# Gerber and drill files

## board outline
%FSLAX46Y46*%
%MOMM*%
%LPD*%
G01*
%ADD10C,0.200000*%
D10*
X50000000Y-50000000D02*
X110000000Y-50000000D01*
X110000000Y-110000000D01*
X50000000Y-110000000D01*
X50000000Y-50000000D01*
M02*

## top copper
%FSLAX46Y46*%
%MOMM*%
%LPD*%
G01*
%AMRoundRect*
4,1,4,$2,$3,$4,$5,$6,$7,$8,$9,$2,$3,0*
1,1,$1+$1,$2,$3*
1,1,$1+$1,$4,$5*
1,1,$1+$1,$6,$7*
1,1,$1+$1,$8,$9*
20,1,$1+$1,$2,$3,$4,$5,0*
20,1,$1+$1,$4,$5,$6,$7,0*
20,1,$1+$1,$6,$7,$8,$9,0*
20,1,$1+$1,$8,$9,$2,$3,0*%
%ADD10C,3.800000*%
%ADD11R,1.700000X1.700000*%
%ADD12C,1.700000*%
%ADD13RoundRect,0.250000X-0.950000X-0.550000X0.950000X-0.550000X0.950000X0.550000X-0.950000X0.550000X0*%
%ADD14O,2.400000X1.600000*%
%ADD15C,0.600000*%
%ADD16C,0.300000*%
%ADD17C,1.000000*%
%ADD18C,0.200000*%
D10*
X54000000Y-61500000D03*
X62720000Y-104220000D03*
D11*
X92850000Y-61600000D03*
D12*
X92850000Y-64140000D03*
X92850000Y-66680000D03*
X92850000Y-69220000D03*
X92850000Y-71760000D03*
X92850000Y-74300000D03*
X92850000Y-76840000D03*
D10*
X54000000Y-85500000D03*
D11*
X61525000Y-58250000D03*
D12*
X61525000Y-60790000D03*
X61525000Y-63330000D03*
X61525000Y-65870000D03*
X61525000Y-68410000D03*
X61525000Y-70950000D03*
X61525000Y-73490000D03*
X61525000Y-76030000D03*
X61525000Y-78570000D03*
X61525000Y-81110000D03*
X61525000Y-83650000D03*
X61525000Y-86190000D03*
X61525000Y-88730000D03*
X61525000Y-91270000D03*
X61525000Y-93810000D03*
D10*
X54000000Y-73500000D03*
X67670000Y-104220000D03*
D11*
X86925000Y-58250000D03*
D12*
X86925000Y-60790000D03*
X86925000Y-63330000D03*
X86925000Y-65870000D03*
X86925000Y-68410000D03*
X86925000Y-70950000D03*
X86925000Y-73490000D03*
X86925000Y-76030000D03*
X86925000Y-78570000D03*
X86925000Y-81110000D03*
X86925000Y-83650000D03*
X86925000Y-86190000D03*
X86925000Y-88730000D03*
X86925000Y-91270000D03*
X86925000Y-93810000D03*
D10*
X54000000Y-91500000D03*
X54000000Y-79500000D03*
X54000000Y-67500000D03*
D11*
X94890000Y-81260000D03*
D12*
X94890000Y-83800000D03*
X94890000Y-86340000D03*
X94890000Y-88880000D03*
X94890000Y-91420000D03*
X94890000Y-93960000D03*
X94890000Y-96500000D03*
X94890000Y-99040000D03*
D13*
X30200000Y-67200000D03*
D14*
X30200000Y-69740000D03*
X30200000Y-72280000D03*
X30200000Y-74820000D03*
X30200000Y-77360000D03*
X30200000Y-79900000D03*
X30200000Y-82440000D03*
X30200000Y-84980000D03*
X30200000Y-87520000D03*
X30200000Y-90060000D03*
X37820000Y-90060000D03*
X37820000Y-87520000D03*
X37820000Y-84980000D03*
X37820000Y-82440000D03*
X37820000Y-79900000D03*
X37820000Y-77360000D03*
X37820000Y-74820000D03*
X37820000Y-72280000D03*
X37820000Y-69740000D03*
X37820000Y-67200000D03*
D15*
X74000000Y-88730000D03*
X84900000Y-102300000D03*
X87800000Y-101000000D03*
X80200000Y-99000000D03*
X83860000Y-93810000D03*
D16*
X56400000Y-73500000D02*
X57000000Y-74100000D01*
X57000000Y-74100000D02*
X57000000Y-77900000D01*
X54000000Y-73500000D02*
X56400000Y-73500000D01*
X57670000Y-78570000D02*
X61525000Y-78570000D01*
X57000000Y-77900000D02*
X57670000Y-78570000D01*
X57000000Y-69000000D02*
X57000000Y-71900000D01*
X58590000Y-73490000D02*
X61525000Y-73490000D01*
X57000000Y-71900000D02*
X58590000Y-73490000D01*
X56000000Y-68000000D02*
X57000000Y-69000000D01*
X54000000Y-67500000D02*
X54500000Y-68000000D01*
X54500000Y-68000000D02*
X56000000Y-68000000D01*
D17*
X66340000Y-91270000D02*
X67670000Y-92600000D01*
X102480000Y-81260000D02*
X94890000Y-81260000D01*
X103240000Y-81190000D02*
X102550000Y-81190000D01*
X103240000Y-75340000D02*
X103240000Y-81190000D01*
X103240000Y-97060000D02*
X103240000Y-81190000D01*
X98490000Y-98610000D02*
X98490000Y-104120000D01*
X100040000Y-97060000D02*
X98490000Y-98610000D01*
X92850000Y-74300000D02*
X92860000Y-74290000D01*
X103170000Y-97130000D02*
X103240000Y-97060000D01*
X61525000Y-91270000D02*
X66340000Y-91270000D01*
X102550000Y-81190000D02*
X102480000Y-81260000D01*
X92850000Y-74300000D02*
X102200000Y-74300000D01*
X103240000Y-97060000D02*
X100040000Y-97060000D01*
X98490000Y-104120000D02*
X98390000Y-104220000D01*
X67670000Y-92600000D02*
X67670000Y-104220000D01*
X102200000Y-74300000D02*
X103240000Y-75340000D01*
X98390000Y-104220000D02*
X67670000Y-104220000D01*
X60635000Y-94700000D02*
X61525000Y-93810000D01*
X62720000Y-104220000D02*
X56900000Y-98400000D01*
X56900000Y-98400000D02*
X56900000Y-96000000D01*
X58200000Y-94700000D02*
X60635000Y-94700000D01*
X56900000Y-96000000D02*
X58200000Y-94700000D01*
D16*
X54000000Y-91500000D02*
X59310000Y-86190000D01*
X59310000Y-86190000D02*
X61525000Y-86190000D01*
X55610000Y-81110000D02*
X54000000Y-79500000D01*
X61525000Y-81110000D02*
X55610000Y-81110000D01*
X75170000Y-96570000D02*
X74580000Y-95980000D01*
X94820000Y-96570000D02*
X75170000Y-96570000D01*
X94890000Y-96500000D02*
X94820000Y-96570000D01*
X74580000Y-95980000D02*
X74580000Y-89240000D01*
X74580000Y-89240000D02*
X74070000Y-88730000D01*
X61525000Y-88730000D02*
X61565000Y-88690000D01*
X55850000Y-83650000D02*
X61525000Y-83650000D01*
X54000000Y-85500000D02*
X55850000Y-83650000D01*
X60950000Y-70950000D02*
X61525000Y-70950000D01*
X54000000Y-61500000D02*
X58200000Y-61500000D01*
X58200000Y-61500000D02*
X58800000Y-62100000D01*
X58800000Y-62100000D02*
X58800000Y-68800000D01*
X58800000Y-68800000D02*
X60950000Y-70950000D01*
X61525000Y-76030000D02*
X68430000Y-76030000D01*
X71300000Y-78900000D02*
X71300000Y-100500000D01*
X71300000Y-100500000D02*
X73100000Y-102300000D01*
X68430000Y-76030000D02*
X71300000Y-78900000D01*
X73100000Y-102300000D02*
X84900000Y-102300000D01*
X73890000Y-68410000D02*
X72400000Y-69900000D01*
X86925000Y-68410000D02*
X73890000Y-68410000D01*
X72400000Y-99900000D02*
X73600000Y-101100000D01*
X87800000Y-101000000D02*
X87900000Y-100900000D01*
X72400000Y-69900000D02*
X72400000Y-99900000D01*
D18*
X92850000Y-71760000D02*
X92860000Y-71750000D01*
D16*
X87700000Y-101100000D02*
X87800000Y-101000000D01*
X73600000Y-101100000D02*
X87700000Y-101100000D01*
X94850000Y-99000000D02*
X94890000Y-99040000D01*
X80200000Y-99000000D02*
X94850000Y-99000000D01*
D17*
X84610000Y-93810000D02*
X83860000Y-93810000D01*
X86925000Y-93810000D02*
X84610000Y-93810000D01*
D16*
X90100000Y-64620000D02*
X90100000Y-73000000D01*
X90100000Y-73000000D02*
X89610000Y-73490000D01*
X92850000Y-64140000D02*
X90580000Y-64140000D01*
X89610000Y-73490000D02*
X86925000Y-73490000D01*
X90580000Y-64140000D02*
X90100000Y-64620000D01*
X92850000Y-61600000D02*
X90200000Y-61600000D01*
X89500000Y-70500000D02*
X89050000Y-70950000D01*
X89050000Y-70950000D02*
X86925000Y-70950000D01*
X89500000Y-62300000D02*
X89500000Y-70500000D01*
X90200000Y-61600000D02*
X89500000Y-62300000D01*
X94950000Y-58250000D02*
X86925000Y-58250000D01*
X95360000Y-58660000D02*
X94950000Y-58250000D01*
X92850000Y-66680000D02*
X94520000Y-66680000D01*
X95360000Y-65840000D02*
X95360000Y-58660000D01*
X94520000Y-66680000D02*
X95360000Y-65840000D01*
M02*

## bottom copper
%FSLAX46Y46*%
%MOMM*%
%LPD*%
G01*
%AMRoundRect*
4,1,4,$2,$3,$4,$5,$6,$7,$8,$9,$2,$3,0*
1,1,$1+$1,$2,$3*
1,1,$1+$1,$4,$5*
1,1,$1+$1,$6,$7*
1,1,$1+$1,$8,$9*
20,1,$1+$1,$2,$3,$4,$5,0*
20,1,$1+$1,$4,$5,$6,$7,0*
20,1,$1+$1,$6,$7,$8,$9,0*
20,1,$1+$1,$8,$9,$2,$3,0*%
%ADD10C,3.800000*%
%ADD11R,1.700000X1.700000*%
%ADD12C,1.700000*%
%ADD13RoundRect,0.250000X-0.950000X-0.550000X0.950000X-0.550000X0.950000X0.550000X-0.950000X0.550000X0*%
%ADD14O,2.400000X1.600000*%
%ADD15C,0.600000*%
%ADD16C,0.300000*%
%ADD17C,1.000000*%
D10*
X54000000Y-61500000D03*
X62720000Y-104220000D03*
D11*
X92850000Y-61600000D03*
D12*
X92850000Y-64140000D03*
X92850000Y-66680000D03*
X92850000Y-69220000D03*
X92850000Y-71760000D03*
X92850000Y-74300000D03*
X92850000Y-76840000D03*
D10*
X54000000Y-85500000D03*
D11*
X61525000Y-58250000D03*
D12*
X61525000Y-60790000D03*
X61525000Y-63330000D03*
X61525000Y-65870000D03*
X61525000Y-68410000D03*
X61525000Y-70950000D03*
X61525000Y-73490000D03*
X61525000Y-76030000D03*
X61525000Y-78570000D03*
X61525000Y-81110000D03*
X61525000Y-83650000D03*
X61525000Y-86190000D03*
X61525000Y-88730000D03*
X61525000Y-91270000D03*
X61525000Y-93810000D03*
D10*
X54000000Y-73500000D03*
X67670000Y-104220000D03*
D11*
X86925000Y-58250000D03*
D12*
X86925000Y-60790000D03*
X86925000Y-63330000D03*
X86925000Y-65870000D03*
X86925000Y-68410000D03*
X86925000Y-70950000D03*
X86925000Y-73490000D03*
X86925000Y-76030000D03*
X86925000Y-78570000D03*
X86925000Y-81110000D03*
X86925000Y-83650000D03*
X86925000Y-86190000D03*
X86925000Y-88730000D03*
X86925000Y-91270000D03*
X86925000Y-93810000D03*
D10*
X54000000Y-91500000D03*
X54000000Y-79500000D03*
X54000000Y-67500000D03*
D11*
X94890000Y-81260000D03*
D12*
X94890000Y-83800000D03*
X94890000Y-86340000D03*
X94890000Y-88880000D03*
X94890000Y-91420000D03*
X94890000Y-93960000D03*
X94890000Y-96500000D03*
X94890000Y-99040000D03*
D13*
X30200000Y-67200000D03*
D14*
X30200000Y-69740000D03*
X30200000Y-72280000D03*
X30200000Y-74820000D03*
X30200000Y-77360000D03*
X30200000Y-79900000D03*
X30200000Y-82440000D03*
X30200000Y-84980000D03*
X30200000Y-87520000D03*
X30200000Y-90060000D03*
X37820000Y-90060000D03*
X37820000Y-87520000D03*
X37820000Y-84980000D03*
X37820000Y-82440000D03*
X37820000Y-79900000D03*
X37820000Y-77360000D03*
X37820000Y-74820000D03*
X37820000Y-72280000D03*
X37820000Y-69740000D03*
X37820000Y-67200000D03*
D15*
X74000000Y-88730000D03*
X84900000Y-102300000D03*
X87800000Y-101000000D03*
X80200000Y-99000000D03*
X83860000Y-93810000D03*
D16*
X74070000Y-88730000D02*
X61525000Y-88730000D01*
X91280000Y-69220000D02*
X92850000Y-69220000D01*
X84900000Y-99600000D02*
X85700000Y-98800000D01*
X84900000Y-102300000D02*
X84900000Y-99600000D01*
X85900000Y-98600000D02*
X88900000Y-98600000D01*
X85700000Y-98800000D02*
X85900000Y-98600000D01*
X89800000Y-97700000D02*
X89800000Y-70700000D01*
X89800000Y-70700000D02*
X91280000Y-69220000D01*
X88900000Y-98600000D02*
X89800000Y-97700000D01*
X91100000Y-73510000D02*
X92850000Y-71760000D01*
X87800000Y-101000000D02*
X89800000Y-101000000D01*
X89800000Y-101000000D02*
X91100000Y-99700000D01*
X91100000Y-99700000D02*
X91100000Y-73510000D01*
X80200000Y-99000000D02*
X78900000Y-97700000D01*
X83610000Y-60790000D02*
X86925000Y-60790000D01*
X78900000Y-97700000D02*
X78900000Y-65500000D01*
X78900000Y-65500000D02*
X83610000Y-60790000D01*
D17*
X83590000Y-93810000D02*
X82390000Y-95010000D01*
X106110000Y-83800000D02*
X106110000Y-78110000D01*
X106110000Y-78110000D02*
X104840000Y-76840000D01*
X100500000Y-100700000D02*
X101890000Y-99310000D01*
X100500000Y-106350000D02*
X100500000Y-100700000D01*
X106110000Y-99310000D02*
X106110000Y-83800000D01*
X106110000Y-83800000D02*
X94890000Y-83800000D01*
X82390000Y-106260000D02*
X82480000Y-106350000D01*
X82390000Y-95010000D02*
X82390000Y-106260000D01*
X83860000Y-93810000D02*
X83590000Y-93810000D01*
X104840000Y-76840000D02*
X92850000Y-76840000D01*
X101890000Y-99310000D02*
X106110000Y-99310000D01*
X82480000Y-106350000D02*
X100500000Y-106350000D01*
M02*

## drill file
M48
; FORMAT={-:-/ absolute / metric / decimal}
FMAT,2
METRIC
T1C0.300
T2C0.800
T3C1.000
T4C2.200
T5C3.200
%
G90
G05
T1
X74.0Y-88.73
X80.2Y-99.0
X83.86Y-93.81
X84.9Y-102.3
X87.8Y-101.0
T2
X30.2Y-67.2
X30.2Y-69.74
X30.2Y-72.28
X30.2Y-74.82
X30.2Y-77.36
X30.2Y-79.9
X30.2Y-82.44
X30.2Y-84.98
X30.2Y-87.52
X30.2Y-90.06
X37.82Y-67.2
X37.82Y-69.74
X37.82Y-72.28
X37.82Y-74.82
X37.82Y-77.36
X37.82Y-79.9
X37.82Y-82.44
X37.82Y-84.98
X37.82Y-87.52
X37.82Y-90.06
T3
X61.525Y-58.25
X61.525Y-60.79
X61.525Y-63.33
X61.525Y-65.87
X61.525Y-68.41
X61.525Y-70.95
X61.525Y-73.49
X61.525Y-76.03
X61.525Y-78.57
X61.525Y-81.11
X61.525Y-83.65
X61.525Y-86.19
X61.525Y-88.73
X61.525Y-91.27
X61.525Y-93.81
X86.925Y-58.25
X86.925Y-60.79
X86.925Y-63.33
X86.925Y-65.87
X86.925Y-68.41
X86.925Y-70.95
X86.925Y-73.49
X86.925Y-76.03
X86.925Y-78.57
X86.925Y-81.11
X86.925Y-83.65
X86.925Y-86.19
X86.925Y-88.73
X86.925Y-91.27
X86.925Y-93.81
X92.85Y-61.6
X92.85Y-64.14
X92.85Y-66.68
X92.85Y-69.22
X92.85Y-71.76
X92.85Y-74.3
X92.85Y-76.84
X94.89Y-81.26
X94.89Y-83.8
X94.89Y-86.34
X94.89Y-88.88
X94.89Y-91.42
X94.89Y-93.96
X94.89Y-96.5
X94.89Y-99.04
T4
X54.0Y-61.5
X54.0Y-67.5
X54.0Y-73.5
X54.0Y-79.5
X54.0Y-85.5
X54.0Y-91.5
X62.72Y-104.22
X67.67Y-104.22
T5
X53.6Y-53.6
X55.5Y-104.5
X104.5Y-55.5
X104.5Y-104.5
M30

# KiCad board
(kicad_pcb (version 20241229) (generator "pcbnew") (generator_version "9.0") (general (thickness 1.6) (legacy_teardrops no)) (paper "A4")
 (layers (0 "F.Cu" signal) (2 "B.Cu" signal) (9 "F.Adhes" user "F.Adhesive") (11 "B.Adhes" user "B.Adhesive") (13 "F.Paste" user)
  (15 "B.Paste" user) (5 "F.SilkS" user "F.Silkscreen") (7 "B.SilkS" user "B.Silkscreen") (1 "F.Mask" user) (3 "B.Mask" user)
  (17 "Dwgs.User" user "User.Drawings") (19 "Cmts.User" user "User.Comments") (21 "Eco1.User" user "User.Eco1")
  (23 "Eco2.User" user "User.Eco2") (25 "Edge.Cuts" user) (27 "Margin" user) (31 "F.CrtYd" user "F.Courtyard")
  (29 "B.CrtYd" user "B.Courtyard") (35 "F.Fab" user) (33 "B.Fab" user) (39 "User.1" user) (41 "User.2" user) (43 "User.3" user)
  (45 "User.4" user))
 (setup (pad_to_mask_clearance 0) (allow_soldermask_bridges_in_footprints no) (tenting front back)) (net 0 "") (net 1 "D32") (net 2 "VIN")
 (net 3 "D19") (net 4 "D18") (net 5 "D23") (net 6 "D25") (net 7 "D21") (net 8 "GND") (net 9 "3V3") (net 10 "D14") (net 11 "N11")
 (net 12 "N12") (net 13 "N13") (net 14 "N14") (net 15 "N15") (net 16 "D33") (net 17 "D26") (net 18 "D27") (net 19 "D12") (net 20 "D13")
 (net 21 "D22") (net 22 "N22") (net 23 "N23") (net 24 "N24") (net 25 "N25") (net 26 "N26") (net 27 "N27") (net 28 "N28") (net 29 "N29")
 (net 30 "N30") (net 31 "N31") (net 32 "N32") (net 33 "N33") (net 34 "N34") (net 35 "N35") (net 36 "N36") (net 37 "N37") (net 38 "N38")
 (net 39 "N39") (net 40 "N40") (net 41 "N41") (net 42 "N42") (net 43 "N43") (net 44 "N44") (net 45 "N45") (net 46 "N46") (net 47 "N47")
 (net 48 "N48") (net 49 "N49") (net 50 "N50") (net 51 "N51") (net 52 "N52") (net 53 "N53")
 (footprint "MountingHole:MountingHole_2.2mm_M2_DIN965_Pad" (layer "F.Cu") (at 54 61.5)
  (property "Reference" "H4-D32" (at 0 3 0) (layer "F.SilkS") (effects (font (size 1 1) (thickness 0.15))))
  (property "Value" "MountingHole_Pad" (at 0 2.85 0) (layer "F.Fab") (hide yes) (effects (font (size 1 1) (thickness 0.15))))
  (pad "1" thru_hole circle (at 0 0) (size 3.8 3.8) (drill 2.2) (layers "*.Cu" "*.Mask") (remove_unused_layers no) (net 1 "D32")
   (zone_connect 2)))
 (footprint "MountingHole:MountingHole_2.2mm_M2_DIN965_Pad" (layer "F.Cu") (at 62.72 104.22)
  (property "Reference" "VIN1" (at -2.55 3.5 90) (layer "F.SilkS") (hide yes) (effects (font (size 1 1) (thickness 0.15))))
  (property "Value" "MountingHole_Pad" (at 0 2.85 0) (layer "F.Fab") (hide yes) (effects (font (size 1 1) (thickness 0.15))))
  (pad "1" thru_hole circle (at 0 0) (size 3.8 3.8) (drill 2.2) (layers "*.Cu" "*.Mask") (remove_unused_layers no) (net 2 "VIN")
   (zone_connect 2)))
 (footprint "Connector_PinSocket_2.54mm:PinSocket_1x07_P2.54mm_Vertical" (layer "F.Cu") (at 92.85 61.6)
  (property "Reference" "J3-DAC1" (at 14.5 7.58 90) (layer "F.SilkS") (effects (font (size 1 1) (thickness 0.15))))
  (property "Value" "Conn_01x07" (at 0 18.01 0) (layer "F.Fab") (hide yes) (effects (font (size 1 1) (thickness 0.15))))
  (pad "1" thru_hole rect (at 0 0) (size 1.7 1.7) (drill 1) (layers "*.Cu" "*.Mask") (remove_unused_layers no) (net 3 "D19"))
  (pad "2" thru_hole circle (at 0 2.54) (size 1.7 1.7) (drill 1) (layers "*.Cu" "*.Mask") (remove_unused_layers no) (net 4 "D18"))
  (pad "3" thru_hole circle (at 0 5.08) (size 1.7 1.7) (drill 1) (layers "*.Cu" "*.Mask") (remove_unused_layers no) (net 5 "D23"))
  (pad "4" thru_hole circle (at 0 7.62) (size 1.7 1.7) (drill 1) (layers "*.Cu" "*.Mask") (remove_unused_layers no) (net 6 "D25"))
  (pad "5" thru_hole circle (at 0 10.16) (size 1.7 1.7) (drill 1) (layers "*.Cu" "*.Mask") (remove_unused_layers no) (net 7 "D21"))
  (pad "6" thru_hole circle (at 0 12.7) (size 1.7 1.7) (drill 1) (layers "*.Cu" "*.Mask") (remove_unused_layers no) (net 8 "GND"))
  (pad "7" thru_hole circle (at 0 15.24) (size 1.7 1.7) (drill 1) (layers "*.Cu" "*.Mask") (remove_unused_layers no) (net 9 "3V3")))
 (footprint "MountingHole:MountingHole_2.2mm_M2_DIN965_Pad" (layer "F.Cu") (at 54 85.5)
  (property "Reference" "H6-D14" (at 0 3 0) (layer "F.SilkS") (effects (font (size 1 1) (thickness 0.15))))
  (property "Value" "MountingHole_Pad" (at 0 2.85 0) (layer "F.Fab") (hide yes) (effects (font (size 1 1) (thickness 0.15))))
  (pad "1" thru_hole circle (at 0 0) (size 3.8 3.8) (drill 2.2) (layers "*.Cu" "*.Mask") (remove_unused_layers no) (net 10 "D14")
   (zone_connect 2)))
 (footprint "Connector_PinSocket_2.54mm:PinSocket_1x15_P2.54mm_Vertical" (layer "F.Cu") (at 61.525 58.25)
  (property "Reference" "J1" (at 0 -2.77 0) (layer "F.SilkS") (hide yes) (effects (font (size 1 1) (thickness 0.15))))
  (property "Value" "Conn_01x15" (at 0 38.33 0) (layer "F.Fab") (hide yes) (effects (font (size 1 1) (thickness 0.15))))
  (pad "1" thru_hole rect (at 0 0) (size 1.7 1.7) (drill 1) (layers "*.Cu" "*.Mask") (remove_unused_layers no) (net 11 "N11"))
  (pad "2" thru_hole circle (at 0 2.54) (size 1.7 1.7) (drill 1) (layers "*.Cu" "*.Mask") (remove_unused_layers no) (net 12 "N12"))
  (pad "3" thru_hole circle (at 0 5.08) (size 1.7 1.7) (drill 1) (layers "*.Cu" "*.Mask") (remove_unused_layers no) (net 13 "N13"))
  (pad "4" thru_hole circle (at 0 7.62) (size 1.7 1.7) (drill 1) (layers "*.Cu" "*.Mask") (remove_unused_layers no) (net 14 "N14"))
  (pad "5" thru_hole circle (at 0 10.16) (size 1.7 1.7) (drill 1) (layers "*.Cu" "*.Mask") (remove_unused_layers no) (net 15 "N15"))
  (pad "6" thru_hole circle (at 0 12.7) (size 1.7 1.7) (drill 1) (layers "*.Cu" "*.Mask") (remove_unused_layers no) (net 1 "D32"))
  (pad "7" thru_hole circle (at 0 15.24) (size 1.7 1.7) (drill 1) (layers "*.Cu" "*.Mask") (remove_unused_layers no) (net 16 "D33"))
  (pad "8" thru_hole circle (at 0 17.78) (size 1.7 1.7) (drill 1) (layers "*.Cu" "*.Mask") (remove_unused_layers no) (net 6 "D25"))
  (pad "9" thru_hole circle (at 0 20.32) (size 1.7 1.7) (drill 1) (layers "*.Cu" "*.Mask") (remove_unused_layers no) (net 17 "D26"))
  (pad "10" thru_hole circle (at 0 22.86) (size 1.7 1.7) (drill 1) (layers "*.Cu" "*.Mask") (remove_unused_layers no) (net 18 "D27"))
  (pad "11" thru_hole circle (at 0 25.4) (size 1.7 1.7) (drill 1) (layers "*.Cu" "*.Mask") (remove_unused_layers no) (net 10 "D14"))
  (pad "12" thru_hole circle (at 0 27.94) (size 1.7 1.7) (drill 1) (layers "*.Cu" "*.Mask") (remove_unused_layers no) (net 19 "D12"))
  (pad "13" thru_hole circle (at 0 30.48) (size 1.7 1.7) (drill 1) (layers "*.Cu" "*.Mask") (remove_unused_layers no) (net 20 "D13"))
  (pad "14" thru_hole circle (at 0 33.02) (size 1.7 1.7) (drill 1) (layers "*.Cu" "*.Mask") (remove_unused_layers no) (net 8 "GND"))
  (pad "15" thru_hole circle (at 0 35.56) (size 1.7 1.7) (drill 1) (layers "*.Cu" "*.Mask") (remove_unused_layers no) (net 2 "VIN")))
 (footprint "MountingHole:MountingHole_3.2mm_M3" (layer "F.Cu") (at 53.6 53.6)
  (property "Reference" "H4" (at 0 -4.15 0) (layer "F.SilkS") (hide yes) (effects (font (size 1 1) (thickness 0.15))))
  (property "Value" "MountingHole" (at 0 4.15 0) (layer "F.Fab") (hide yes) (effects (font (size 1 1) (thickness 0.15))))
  (pad "" np_thru_hole circle (at 0 0) (size 3.2 3.2) (drill 3.2) (layers "*.Cu" "*.Mask")))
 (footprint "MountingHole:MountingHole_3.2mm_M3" (layer "F.Cu") (at 55.5 104.5)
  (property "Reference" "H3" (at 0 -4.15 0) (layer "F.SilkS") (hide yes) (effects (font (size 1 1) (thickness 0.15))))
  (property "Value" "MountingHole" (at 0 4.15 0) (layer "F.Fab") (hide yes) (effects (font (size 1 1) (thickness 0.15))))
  (pad "" np_thru_hole circle (at 0 0) (size 3.2 3.2) (drill 3.2) (layers "*.Cu" "*.Mask")))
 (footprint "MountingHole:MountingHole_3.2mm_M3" (layer "F.Cu") (at 104.5 55.5)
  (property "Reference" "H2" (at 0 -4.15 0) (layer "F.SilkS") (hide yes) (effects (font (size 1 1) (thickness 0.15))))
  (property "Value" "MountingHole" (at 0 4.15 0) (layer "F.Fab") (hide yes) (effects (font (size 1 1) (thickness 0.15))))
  (pad "" np_thru_hole circle (at 0 0) (size 3.2 3.2) (drill 3.2) (layers "*.Cu" "*.Mask")))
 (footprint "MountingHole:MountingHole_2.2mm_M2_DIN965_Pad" (layer "F.Cu") (at 54 73.5)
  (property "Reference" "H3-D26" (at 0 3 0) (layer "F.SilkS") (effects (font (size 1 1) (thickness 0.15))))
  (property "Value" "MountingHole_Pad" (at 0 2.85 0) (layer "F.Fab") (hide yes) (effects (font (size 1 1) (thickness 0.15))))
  (pad "1" thru_hole circle (at 0 0) (size 3.8 3.8) (drill 2.2) (layers "*.Cu" "*.Mask") (remove_unused_layers no) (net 17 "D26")
   (zone_connect 2)))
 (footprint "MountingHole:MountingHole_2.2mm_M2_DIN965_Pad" (layer "F.Cu") (at 67.67 104.22)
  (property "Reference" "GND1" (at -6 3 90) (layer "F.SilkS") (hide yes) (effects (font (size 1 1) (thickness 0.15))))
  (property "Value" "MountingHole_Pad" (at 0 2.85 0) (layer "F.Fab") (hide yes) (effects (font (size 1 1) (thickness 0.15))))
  (pad "1" thru_hole circle (at 0 0) (size 3.8 3.8) (drill 2.2) (layers "*.Cu" "*.Mask") (remove_unused_layers no) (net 8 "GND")
   (zone_connect 2)))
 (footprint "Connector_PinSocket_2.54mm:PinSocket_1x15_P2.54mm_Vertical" (layer "F.Cu") (at 86.925 58.25)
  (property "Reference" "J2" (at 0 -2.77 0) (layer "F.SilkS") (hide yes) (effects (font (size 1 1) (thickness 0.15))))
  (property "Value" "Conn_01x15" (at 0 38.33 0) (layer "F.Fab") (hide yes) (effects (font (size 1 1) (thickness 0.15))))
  (pad "1" thru_hole rect (at 0 0) (size 1.7 1.7) (drill 1) (layers "*.Cu" "*.Mask") (remove_unused_layers no) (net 5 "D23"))
  (pad "2" thru_hole circle (at 0 2.54) (size 1.7 1.7) (drill 1) (layers "*.Cu" "*.Mask") (remove_unused_layers no) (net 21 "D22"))
  (pad "3" thru_hole circle (at 0 5.08) (size 1.7 1.7) (drill 1) (layers "*.Cu" "*.Mask") (remove_unused_layers no) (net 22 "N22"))
  (pad "4" thru_hole circle (at 0 7.62) (size 1.7 1.7) (drill 1) (layers "*.Cu" "*.Mask") (remove_unused_layers no) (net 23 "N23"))
  (pad "5" thru_hole circle (at 0 10.16) (size 1.7 1.7) (drill 1) (layers "*.Cu" "*.Mask") (remove_unused_layers no) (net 7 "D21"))
  (pad "6" thru_hole circle (at 0 12.7) (size 1.7 1.7) (drill 1) (layers "*.Cu" "*.Mask") (remove_unused_layers no) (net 3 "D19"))
  (pad "7" thru_hole circle (at 0 15.24) (size 1.7 1.7) (drill 1) (layers "*.Cu" "*.Mask") (remove_unused_layers no) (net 4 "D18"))
  (pad "8" thru_hole circle (at 0 17.78) (size 1.7 1.7) (drill 1) (layers "*.Cu" "*.Mask") (remove_unused_layers no) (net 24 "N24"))
  (pad "9" thru_hole circle (at 0 20.32) (size 1.7 1.7) (drill 1) (layers "*.Cu" "*.Mask") (remove_unused_layers no) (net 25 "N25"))
  (pad "10" thru_hole circle (at 0 22.86) (size 1.7 1.7) (drill 1) (layers "*.Cu" "*.Mask") (remove_unused_layers no) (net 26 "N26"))
  (pad "11" thru_hole circle (at 0 25.4) (size 1.7 1.7) (drill 1) (layers "*.Cu" "*.Mask") (remove_unused_layers no) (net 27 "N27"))
  (pad "12" thru_hole circle (at 0 27.94) (size 1.7 1.7) (drill 1) (layers "*.Cu" "*.Mask") (remove_unused_layers no) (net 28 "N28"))
  (pad "13" thru_hole circle (at 0 30.48) (size 1.7 1.7) (drill 1) (layers "*.Cu" "*.Mask") (remove_unused_layers no) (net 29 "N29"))
  (pad "14" thru_hole circle (at 0 33.02) (size 1.7 1.7) (drill 1) (layers "*.Cu" "*.Mask") (remove_unused_layers no) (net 8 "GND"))
  (pad "15" thru_hole circle (at 0 35.56) (size 1.7 1.7) (drill 1) (layers "*.Cu" "*.Mask") (remove_unused_layers no) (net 9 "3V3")))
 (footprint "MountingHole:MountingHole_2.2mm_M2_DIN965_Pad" (layer "F.Cu") (at 54 91.5)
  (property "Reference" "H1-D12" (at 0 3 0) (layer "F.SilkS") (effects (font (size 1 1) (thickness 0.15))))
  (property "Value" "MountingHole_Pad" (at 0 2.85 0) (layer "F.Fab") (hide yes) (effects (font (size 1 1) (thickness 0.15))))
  (pad "1" thru_hole circle (at 0 0) (size 3.8 3.8) (drill 2.2) (layers "*.Cu" "*.Mask") (remove_unused_layers no) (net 19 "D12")
   (zone_connect 2)))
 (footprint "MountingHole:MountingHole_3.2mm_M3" (layer "F.Cu") (at 104.5 104.5)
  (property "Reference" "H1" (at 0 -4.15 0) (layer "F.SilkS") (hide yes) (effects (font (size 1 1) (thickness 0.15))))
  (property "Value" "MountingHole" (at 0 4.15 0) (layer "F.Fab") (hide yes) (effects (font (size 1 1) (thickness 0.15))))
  (pad "" np_thru_hole circle (at 0 0) (size 3.2 3.2) (drill 3.2) (layers "*.Cu" "*.Mask")))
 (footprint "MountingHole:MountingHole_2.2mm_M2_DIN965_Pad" (layer "F.Cu") (at 54 79.5)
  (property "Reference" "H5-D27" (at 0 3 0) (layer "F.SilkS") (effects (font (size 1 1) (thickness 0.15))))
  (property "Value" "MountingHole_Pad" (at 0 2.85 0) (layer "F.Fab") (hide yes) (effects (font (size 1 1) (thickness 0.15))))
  (pad "1" thru_hole circle (at 0 0) (size 3.8 3.8) (drill 2.2) (layers "*.Cu" "*.Mask") (remove_unused_layers no) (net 18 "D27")
   (zone_connect 2)))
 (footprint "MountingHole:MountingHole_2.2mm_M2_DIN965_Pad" (layer "F.Cu") (at 54 67.5)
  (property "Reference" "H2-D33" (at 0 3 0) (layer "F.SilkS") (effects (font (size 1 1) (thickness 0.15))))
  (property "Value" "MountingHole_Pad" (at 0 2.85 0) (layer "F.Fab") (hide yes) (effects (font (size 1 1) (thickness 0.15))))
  (pad "1" thru_hole circle (at 0 0) (size 3.8 3.8) (drill 2.2) (layers "*.Cu" "*.Mask") (remove_unused_layers no) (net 16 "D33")
   (zone_connect 2)))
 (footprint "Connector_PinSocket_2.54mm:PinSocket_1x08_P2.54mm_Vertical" (layer "F.Cu") (at 94.89 81.26)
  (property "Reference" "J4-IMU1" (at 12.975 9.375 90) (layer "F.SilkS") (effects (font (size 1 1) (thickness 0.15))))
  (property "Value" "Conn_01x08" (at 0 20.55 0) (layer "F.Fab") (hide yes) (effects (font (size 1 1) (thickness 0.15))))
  (pad "1" thru_hole rect (at 0 0) (size 1.7 1.7) (drill 1) (layers "*.Cu" "*.Mask") (remove_unused_layers no) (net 8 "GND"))
  (pad "2" thru_hole circle (at 0 2.54) (size 1.7 1.7) (drill 1) (layers "*.Cu" "*.Mask") (remove_unused_layers no) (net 9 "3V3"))
  (pad "3" thru_hole circle (at 0 5.08) (size 1.7 1.7) (drill 1) (layers "*.Cu" "*.Mask") (remove_unused_layers no) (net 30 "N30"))
  (pad "4" thru_hole circle (at 0 7.62) (size 1.7 1.7) (drill 1) (layers "*.Cu" "*.Mask") (remove_unused_layers no) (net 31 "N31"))
  (pad "5" thru_hole circle (at 0 10.16) (size 1.7 1.7) (drill 1) (layers "*.Cu" "*.Mask") (remove_unused_layers no) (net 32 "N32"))
  (pad "6" thru_hole circle (at 0 12.7) (size 1.7 1.7) (drill 1) (layers "*.Cu" "*.Mask") (remove_unused_layers no) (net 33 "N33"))
  (pad "7" thru_hole circle (at 0 15.24) (size 1.7 1.7) (drill 1) (layers "*.Cu" "*.Mask") (remove_unused_layers no) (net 20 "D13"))
  (pad "8" thru_hole circle (at 0 17.78) (size 1.7 1.7) (drill 1) (layers "*.Cu" "*.Mask") (remove_unused_layers no) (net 21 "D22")))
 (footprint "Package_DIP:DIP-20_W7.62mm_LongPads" (layer "F.Cu") (at 30.2 67.2)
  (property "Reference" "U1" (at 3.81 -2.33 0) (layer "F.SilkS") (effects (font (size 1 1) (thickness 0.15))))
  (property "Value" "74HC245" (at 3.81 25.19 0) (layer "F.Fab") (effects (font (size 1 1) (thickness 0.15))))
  (pad "1" thru_hole roundrect (at 0 0) (size 2.4 1.6) (drill 0.8) (layers "*.Cu" "*.Mask") (remove_unused_layers no)
   (roundrect_rratio 0.15625) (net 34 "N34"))
  (pad "2" thru_hole oval (at 0 2.54) (size 2.4 1.6) (drill 0.8) (layers "*.Cu" "*.Mask") (remove_unused_layers no) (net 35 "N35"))
  (pad "3" thru_hole oval (at 0 5.08) (size 2.4 1.6) (drill 0.8) (layers "*.Cu" "*.Mask") (remove_unused_layers no) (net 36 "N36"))
  (pad "4" thru_hole oval (at 0 7.62) (size 2.4 1.6) (drill 0.8) (layers "*.Cu" "*.Mask") (remove_unused_layers no) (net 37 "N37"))
  (pad "5" thru_hole oval (at 0 10.16) (size 2.4 1.6) (drill 0.8) (layers "*.Cu" "*.Mask") (remove_unused_layers no) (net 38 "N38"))
  (pad "6" thru_hole oval (at 0 12.7) (size 2.4 1.6) (drill 0.8) (layers "*.Cu" "*.Mask") (remove_unused_layers no) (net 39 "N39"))
  (pad "7" thru_hole oval (at 0 15.24) (size 2.4 1.6) (drill 0.8) (layers "*.Cu" "*.Mask") (remove_unused_layers no) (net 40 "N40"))
  (pad "8" thru_hole oval (at 0 17.78) (size 2.4 1.6) (drill 0.8) (layers "*.Cu" "*.Mask") (remove_unused_layers no) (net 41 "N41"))
  (pad "9" thru_hole oval (at 0 20.32) (size 2.4 1.6) (drill 0.8) (layers "*.Cu" "*.Mask") (remove_unused_layers no) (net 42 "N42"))
  (pad "10" thru_hole oval (at 0 22.86) (size 2.4 1.6) (drill 0.8) (layers "*.Cu" "*.Mask") (remove_unused_layers no) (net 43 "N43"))
  (pad "11" thru_hole oval (at 7.62 22.86) (size 2.4 1.6) (drill 0.8) (layers "*.Cu" "*.Mask") (remove_unused_layers no) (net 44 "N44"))
  (pad "12" thru_hole oval (at 7.62 20.32) (size 2.4 1.6) (drill 0.8) (layers "*.Cu" "*.Mask") (remove_unused_layers no) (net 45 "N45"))
  (pad "13" thru_hole oval (at 7.62 17.78) (size 2.4 1.6) (drill 0.8) (layers "*.Cu" "*.Mask") (remove_unused_layers no) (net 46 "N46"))
  (pad "14" thru_hole oval (at 7.62 15.24) (size 2.4 1.6) (drill 0.8) (layers "*.Cu" "*.Mask") (remove_unused_layers no) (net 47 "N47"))
  (pad "15" thru_hole oval (at 7.62 12.7) (size 2.4 1.6) (drill 0.8) (layers "*.Cu" "*.Mask") (remove_unused_layers no) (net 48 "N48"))
  (pad "16" thru_hole oval (at 7.62 10.16) (size 2.4 1.6) (drill 0.8) (layers "*.Cu" "*.Mask") (remove_unused_layers no) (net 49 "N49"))
  (pad "17" thru_hole oval (at 7.62 7.62) (size 2.4 1.6) (drill 0.8) (layers "*.Cu" "*.Mask") (remove_unused_layers no) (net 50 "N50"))
  (pad "18" thru_hole oval (at 7.62 5.08) (size 2.4 1.6) (drill 0.8) (layers "*.Cu" "*.Mask") (remove_unused_layers no) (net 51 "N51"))
  (pad "19" thru_hole oval (at 7.62 2.54) (size 2.4 1.6) (drill 0.8) (layers "*.Cu" "*.Mask") (remove_unused_layers no) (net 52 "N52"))
  (pad "20" thru_hole oval (at 7.62 0) (size 2.4 1.6) (drill 0.8) (layers "*.Cu" "*.Mask") (remove_unused_layers no) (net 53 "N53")))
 (gr_rect (start 50 50) (end 110 110) (stroke (width 0.2) (type solid)) (fill no) (layer "Edge.Cuts"))
 (segment (start 56.4 73.5) (end 57 74.1) (width 0.3) (layer "F.Cu") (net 17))
 (segment (start 57 74.1) (end 57 77.9) (width 0.3) (layer "F.Cu") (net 17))
 (segment (start 54 73.5) (end 56.4 73.5) (width 0.3) (layer "F.Cu") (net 17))
 (segment (start 57.67 78.57) (end 61.525 78.57) (width 0.3) (layer "F.Cu") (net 17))
 (segment (start 57 77.9) (end 57.67 78.57) (width 0.3) (layer "F.Cu") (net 17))
 (segment (start 57 69) (end 57 71.9) (width 0.3) (layer "F.Cu") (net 16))
 (segment (start 58.59 73.49) (end 61.525 73.49) (width 0.3) (layer "F.Cu") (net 16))
 (segment (start 57 71.9) (end 58.59 73.49) (width 0.3) (layer "F.Cu") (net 16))
 (segment (start 56 68) (end 57 69) (width 0.3) (layer "F.Cu") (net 16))
 (segment (start 54 67.5) (end 54.5 68) (width 0.3) (layer "F.Cu") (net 16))
 (segment (start 54.5 68) (end 56 68) (width 0.3) (layer "F.Cu") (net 16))
 (segment (start 66.34 91.27) (end 67.67 92.6) (width 1) (layer "F.Cu") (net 8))
 (segment (start 102.48 81.26) (end 94.89 81.26) (width 1) (layer "F.Cu") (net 8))
 (segment (start 103.24 81.19) (end 102.55 81.19) (width 1) (layer "F.Cu") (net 8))
 (segment (start 103.24 75.34) (end 103.24 81.19) (width 1) (layer "F.Cu") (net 8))
 (segment (start 103.24 97.06) (end 103.24 81.19) (width 1) (layer "F.Cu") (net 8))
 (segment (start 98.49 98.61) (end 98.49 104.12) (width 1) (layer "F.Cu") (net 8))
 (segment (start 100.04 97.06) (end 98.49 98.61) (width 1) (layer "F.Cu") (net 8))
 (segment (start 92.85 74.3) (end 92.86 74.29) (width 1) (layer "F.Cu") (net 8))
 (segment (start 103.17 97.13) (end 103.24 97.06) (width 1) (layer "F.Cu") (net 8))
 (segment (start 61.525 91.27) (end 66.34 91.27) (width 1) (layer "F.Cu") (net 8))
 (segment (start 102.55 81.19) (end 102.48 81.26) (width 1) (layer "F.Cu") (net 8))
 (segment (start 92.85 74.3) (end 102.2 74.3) (width 1) (layer "F.Cu") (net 8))
 (segment (start 103.24 97.06) (end 100.04 97.06) (width 1) (layer "F.Cu") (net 8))
 (segment (start 98.49 104.12) (end 98.39 104.22) (width 1) (layer "F.Cu") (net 8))
 (segment (start 67.67 92.6) (end 67.67 104.22) (width 1) (layer "F.Cu") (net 8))
 (segment (start 102.2 74.3) (end 103.24 75.34) (width 1) (layer "F.Cu") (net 8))
 (segment (start 98.39 104.22) (end 67.67 104.22) (width 1) (layer "F.Cu") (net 8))
 (segment (start 60.635 94.7) (end 61.525 93.81) (width 1) (layer "F.Cu") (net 2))
 (segment (start 62.72 104.22) (end 56.9 98.4) (width 1) (layer "F.Cu") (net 2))
 (segment (start 56.9 98.4) (end 56.9 96) (width 1) (layer "F.Cu") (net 2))
 (segment (start 58.2 94.7) (end 60.635 94.7) (width 1) (layer "F.Cu") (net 2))
 (segment (start 56.9 96) (end 58.2 94.7) (width 1) (layer "F.Cu") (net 2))
 (segment (start 54 91.5) (end 59.31 86.19) (width 0.3) (layer "F.Cu") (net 19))
 (segment (start 59.31 86.19) (end 61.525 86.19) (width 0.3) (layer "F.Cu") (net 19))
 (segment (start 55.61 81.11) (end 54 79.5) (width 0.3) (layer "F.Cu") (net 18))
 (segment (start 61.525 81.11) (end 55.61 81.11) (width 0.3) (layer "F.Cu") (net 18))
 (segment (start 75.17 96.57) (end 74.58 95.98) (width 0.3) (layer "F.Cu") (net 20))
 (segment (start 94.82 96.57) (end 75.17 96.57) (width 0.3) (layer "F.Cu") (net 20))
 (segment (start 94.89 96.5) (end 94.82 96.57) (width 0.3) (layer "F.Cu") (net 20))
 (segment (start 74.58 95.98) (end 74.58 89.24) (width 0.3) (layer "F.Cu") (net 20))
 (segment (start 74.58 89.24) (end 74.07 88.73) (width 0.3) (layer "F.Cu") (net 20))
 (segment (start 61.525 88.73) (end 61.565 88.69) (width 0.3) (layer "F.Cu") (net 20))
 (via (at 74 88.73) (size 0.6) (drill 0.3) (layers "F.Cu" "B.Cu") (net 20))
 (segment (start 74.07 88.73) (end 61.525 88.73) (width 0.3) (layer "B.Cu") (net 20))
 (segment (start 55.85 83.65) (end 61.525 83.65) (width 0.3) (layer "F.Cu") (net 10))
 (segment (start 54 85.5) (end 55.85 83.65) (width 0.3) (layer "F.Cu") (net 10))
 (segment (start 60.95 70.95) (end 61.525 70.95) (width 0.3) (layer "F.Cu") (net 1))
 (segment (start 54 61.5) (end 58.2 61.5) (width 0.3) (layer "F.Cu") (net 1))
 (segment (start 58.2 61.5) (end 58.8 62.1) (width 0.3) (layer "F.Cu") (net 1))
 (segment (start 58.8 62.1) (end 58.8 68.8) (width 0.3) (layer "F.Cu") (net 1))
 (segment (start 58.8 68.8) (end 60.95 70.95) (width 0.3) (layer "F.Cu") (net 1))
 (segment (start 61.525 76.03) (end 68.43 76.03) (width 0.3) (layer "F.Cu") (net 6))
 (segment (start 71.3 78.9) (end 71.3 100.5) (width 0.3) (layer "F.Cu") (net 6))
 (segment (start 71.3 100.5) (end 73.1 102.3) (width 0.3) (layer "F.Cu") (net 6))
 (segment (start 68.43 76.03) (end 71.3 78.9) (width 0.3) (layer "F.Cu") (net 6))
 (segment (start 73.1 102.3) (end 84.9 102.3) (width 0.3) (layer "F.Cu") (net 6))
 (via (at 84.9 102.3) (size 0.6) (drill 0.3) (layers "F.Cu" "B.Cu") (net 6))
 (segment (start 91.28 69.22) (end 92.85 69.22) (width 0.3) (layer "B.Cu") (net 6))
 (segment (start 84.9 99.6) (end 85.7 98.8) (width 0.3) (layer "B.Cu") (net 6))
 (segment (start 84.9 102.3) (end 84.9 99.6) (width 0.3) (layer "B.Cu") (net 6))
 (segment (start 85.9 98.6) (end 88.9 98.6) (width 0.3) (layer "B.Cu") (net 6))
 (segment (start 85.7 98.8) (end 85.9 98.6) (width 0.3) (layer "B.Cu") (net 6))
 (segment (start 89.8 97.7) (end 89.8 70.7) (width 0.3) (layer "B.Cu") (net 6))
 (segment (start 89.8 70.7) (end 91.28 69.22) (width 0.3) (layer "B.Cu") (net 6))
 (segment (start 88.9 98.6) (end 89.8 97.7) (width 0.3) (layer "B.Cu") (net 6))
 (segment (start 73.89 68.41) (end 72.4 69.9) (width 0.3) (layer "F.Cu") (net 7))
 (segment (start 86.925 68.41) (end 73.89 68.41) (width 0.3) (layer "F.Cu") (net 7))
 (segment (start 72.4 99.9) (end 73.6 101.1) (width 0.3) (layer "F.Cu") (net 7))
 (segment (start 87.8 101) (end 87.9 100.9) (width 0.3) (layer "F.Cu") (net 7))
 (segment (start 72.4 69.9) (end 72.4 99.9) (width 0.3) (layer "F.Cu") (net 7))
 (segment (start 92.85 71.76) (end 92.86 71.75) (width 0.2) (layer "F.Cu") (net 7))
 (segment (start 87.7 101.1) (end 87.8 101) (width 0.3) (layer "F.Cu") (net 7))
 (segment (start 73.6 101.1) (end 87.7 101.1) (width 0.3) (layer "F.Cu") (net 7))
 (via (at 87.8 101) (size 0.6) (drill 0.3) (layers "F.Cu" "B.Cu") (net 7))
 (segment (start 91.1 73.51) (end 92.85 71.76) (width 0.3) (layer "B.Cu") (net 7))
 (segment (start 87.8 101) (end 89.8 101) (width 0.3) (layer "B.Cu") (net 7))
 (segment (start 89.8 101) (end 91.1 99.7) (width 0.3) (layer "B.Cu") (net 7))
 (segment (start 91.1 99.7) (end 91.1 73.51) (width 0.3) (layer "B.Cu") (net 7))
 (segment (start 94.85 99) (end 94.89 99.04) (width 0.3) (layer "F.Cu") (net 21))
 (segment (start 80.2 99) (end 94.85 99) (width 0.3) (layer "F.Cu") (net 21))
 (via (at 80.2 99) (size 0.6) (drill 0.3) (layers "F.Cu" "B.Cu") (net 21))
 (segment (start 80.2 99) (end 78.9 97.7) (width 0.3) (layer "B.Cu") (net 21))
 (segment (start 83.61 60.79) (end 86.925 60.79) (width 0.3) (layer "B.Cu") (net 21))
 (segment (start 78.9 97.7) (end 78.9 65.5) (width 0.3) (layer "B.Cu") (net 21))
 (segment (start 78.9 65.5) (end 83.61 60.79) (width 0.3) (layer "B.Cu") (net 21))
 (segment (start 84.61 93.81) (end 83.86 93.81) (width 1) (layer "F.Cu") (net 9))
 (segment (start 86.925 93.81) (end 84.61 93.81) (width 1) (layer "F.Cu") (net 9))
 (via (at 83.86 93.81) (size 0.6) (drill 0.3) (layers "F.Cu" "B.Cu") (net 9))
 (segment (start 83.59 93.81) (end 82.39 95.01) (width 1) (layer "B.Cu") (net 9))
 (segment (start 106.11 83.8) (end 106.11 78.11) (width 1) (layer "B.Cu") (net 9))
 (segment (start 106.11 78.11) (end 104.84 76.84) (width 1) (layer "B.Cu") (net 9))
 (segment (start 100.5 100.7) (end 101.89 99.31) (width 1) (layer "B.Cu") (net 9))
 (segment (start 100.5 106.35) (end 100.5 100.7) (width 1) (layer "B.Cu") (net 9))
 (segment (start 106.11 99.31) (end 106.11 83.8) (width 1) (layer "B.Cu") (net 9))
 (segment (start 106.11 83.8) (end 94.89 83.8) (width 1) (layer "B.Cu") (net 9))
 (segment (start 82.39 106.26) (end 82.48 106.35) (width 1) (layer "B.Cu") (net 9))
 (segment (start 82.39 95.01) (end 82.39 106.26) (width 1) (layer "B.Cu") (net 9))
 (segment (start 83.86 93.81) (end 83.59 93.81) (width 1) (layer "B.Cu") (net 9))
 (segment (start 104.84 76.84) (end 92.85 76.84) (width 1) (layer "B.Cu") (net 9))
 (segment (start 101.89 99.31) (end 106.11 99.31) (width 1) (layer "B.Cu") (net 9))
 (segment (start 82.48 106.35) (end 100.5 106.35) (width 1) (layer "B.Cu") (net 9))
 (segment (start 90.1 64.62) (end 90.1 73) (width 0.3) (layer "F.Cu") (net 4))
 (segment (start 90.1 73) (end 89.61 73.49) (width 0.3) (layer "F.Cu") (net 4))
 (segment (start 92.85 64.14) (end 90.58 64.14) (width 0.3) (layer "F.Cu") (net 4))
 (segment (start 89.61 73.49) (end 86.925 73.49) (width 0.3) (layer "F.Cu") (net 4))
 (segment (start 90.58 64.14) (end 90.1 64.62) (width 0.3) (layer "F.Cu") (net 4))
 (segment (start 92.85 61.6) (end 90.2 61.6) (width 0.3) (layer "F.Cu") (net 3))
 (segment (start 89.5 70.5) (end 89.05 70.95) (width 0.3) (layer "F.Cu") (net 3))
 (segment (start 89.05 70.95) (end 86.925 70.95) (width 0.3) (layer "F.Cu") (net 3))
 (segment (start 89.5 62.3) (end 89.5 70.5) (width 0.3) (layer "F.Cu") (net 3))
 (segment (start 90.2 61.6) (end 89.5 62.3) (width 0.3) (layer "F.Cu") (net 3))
 (segment (start 94.95 58.25) (end 86.925 58.25) (width 0.3) (layer "F.Cu") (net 5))
 (segment (start 95.36 58.66) (end 94.95 58.25) (width 0.3) (layer "F.Cu") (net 5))
 (segment (start 92.85 66.68) (end 94.52 66.68) (width 0.3) (layer "F.Cu") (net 5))
 (segment (start 95.36 65.84) (end 95.36 58.66) (width 0.3) (layer "F.Cu") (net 5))
 (segment (start 94.52 66.68) (end 95.36 65.84) (width 0.3) (layer "F.Cu") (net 5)))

